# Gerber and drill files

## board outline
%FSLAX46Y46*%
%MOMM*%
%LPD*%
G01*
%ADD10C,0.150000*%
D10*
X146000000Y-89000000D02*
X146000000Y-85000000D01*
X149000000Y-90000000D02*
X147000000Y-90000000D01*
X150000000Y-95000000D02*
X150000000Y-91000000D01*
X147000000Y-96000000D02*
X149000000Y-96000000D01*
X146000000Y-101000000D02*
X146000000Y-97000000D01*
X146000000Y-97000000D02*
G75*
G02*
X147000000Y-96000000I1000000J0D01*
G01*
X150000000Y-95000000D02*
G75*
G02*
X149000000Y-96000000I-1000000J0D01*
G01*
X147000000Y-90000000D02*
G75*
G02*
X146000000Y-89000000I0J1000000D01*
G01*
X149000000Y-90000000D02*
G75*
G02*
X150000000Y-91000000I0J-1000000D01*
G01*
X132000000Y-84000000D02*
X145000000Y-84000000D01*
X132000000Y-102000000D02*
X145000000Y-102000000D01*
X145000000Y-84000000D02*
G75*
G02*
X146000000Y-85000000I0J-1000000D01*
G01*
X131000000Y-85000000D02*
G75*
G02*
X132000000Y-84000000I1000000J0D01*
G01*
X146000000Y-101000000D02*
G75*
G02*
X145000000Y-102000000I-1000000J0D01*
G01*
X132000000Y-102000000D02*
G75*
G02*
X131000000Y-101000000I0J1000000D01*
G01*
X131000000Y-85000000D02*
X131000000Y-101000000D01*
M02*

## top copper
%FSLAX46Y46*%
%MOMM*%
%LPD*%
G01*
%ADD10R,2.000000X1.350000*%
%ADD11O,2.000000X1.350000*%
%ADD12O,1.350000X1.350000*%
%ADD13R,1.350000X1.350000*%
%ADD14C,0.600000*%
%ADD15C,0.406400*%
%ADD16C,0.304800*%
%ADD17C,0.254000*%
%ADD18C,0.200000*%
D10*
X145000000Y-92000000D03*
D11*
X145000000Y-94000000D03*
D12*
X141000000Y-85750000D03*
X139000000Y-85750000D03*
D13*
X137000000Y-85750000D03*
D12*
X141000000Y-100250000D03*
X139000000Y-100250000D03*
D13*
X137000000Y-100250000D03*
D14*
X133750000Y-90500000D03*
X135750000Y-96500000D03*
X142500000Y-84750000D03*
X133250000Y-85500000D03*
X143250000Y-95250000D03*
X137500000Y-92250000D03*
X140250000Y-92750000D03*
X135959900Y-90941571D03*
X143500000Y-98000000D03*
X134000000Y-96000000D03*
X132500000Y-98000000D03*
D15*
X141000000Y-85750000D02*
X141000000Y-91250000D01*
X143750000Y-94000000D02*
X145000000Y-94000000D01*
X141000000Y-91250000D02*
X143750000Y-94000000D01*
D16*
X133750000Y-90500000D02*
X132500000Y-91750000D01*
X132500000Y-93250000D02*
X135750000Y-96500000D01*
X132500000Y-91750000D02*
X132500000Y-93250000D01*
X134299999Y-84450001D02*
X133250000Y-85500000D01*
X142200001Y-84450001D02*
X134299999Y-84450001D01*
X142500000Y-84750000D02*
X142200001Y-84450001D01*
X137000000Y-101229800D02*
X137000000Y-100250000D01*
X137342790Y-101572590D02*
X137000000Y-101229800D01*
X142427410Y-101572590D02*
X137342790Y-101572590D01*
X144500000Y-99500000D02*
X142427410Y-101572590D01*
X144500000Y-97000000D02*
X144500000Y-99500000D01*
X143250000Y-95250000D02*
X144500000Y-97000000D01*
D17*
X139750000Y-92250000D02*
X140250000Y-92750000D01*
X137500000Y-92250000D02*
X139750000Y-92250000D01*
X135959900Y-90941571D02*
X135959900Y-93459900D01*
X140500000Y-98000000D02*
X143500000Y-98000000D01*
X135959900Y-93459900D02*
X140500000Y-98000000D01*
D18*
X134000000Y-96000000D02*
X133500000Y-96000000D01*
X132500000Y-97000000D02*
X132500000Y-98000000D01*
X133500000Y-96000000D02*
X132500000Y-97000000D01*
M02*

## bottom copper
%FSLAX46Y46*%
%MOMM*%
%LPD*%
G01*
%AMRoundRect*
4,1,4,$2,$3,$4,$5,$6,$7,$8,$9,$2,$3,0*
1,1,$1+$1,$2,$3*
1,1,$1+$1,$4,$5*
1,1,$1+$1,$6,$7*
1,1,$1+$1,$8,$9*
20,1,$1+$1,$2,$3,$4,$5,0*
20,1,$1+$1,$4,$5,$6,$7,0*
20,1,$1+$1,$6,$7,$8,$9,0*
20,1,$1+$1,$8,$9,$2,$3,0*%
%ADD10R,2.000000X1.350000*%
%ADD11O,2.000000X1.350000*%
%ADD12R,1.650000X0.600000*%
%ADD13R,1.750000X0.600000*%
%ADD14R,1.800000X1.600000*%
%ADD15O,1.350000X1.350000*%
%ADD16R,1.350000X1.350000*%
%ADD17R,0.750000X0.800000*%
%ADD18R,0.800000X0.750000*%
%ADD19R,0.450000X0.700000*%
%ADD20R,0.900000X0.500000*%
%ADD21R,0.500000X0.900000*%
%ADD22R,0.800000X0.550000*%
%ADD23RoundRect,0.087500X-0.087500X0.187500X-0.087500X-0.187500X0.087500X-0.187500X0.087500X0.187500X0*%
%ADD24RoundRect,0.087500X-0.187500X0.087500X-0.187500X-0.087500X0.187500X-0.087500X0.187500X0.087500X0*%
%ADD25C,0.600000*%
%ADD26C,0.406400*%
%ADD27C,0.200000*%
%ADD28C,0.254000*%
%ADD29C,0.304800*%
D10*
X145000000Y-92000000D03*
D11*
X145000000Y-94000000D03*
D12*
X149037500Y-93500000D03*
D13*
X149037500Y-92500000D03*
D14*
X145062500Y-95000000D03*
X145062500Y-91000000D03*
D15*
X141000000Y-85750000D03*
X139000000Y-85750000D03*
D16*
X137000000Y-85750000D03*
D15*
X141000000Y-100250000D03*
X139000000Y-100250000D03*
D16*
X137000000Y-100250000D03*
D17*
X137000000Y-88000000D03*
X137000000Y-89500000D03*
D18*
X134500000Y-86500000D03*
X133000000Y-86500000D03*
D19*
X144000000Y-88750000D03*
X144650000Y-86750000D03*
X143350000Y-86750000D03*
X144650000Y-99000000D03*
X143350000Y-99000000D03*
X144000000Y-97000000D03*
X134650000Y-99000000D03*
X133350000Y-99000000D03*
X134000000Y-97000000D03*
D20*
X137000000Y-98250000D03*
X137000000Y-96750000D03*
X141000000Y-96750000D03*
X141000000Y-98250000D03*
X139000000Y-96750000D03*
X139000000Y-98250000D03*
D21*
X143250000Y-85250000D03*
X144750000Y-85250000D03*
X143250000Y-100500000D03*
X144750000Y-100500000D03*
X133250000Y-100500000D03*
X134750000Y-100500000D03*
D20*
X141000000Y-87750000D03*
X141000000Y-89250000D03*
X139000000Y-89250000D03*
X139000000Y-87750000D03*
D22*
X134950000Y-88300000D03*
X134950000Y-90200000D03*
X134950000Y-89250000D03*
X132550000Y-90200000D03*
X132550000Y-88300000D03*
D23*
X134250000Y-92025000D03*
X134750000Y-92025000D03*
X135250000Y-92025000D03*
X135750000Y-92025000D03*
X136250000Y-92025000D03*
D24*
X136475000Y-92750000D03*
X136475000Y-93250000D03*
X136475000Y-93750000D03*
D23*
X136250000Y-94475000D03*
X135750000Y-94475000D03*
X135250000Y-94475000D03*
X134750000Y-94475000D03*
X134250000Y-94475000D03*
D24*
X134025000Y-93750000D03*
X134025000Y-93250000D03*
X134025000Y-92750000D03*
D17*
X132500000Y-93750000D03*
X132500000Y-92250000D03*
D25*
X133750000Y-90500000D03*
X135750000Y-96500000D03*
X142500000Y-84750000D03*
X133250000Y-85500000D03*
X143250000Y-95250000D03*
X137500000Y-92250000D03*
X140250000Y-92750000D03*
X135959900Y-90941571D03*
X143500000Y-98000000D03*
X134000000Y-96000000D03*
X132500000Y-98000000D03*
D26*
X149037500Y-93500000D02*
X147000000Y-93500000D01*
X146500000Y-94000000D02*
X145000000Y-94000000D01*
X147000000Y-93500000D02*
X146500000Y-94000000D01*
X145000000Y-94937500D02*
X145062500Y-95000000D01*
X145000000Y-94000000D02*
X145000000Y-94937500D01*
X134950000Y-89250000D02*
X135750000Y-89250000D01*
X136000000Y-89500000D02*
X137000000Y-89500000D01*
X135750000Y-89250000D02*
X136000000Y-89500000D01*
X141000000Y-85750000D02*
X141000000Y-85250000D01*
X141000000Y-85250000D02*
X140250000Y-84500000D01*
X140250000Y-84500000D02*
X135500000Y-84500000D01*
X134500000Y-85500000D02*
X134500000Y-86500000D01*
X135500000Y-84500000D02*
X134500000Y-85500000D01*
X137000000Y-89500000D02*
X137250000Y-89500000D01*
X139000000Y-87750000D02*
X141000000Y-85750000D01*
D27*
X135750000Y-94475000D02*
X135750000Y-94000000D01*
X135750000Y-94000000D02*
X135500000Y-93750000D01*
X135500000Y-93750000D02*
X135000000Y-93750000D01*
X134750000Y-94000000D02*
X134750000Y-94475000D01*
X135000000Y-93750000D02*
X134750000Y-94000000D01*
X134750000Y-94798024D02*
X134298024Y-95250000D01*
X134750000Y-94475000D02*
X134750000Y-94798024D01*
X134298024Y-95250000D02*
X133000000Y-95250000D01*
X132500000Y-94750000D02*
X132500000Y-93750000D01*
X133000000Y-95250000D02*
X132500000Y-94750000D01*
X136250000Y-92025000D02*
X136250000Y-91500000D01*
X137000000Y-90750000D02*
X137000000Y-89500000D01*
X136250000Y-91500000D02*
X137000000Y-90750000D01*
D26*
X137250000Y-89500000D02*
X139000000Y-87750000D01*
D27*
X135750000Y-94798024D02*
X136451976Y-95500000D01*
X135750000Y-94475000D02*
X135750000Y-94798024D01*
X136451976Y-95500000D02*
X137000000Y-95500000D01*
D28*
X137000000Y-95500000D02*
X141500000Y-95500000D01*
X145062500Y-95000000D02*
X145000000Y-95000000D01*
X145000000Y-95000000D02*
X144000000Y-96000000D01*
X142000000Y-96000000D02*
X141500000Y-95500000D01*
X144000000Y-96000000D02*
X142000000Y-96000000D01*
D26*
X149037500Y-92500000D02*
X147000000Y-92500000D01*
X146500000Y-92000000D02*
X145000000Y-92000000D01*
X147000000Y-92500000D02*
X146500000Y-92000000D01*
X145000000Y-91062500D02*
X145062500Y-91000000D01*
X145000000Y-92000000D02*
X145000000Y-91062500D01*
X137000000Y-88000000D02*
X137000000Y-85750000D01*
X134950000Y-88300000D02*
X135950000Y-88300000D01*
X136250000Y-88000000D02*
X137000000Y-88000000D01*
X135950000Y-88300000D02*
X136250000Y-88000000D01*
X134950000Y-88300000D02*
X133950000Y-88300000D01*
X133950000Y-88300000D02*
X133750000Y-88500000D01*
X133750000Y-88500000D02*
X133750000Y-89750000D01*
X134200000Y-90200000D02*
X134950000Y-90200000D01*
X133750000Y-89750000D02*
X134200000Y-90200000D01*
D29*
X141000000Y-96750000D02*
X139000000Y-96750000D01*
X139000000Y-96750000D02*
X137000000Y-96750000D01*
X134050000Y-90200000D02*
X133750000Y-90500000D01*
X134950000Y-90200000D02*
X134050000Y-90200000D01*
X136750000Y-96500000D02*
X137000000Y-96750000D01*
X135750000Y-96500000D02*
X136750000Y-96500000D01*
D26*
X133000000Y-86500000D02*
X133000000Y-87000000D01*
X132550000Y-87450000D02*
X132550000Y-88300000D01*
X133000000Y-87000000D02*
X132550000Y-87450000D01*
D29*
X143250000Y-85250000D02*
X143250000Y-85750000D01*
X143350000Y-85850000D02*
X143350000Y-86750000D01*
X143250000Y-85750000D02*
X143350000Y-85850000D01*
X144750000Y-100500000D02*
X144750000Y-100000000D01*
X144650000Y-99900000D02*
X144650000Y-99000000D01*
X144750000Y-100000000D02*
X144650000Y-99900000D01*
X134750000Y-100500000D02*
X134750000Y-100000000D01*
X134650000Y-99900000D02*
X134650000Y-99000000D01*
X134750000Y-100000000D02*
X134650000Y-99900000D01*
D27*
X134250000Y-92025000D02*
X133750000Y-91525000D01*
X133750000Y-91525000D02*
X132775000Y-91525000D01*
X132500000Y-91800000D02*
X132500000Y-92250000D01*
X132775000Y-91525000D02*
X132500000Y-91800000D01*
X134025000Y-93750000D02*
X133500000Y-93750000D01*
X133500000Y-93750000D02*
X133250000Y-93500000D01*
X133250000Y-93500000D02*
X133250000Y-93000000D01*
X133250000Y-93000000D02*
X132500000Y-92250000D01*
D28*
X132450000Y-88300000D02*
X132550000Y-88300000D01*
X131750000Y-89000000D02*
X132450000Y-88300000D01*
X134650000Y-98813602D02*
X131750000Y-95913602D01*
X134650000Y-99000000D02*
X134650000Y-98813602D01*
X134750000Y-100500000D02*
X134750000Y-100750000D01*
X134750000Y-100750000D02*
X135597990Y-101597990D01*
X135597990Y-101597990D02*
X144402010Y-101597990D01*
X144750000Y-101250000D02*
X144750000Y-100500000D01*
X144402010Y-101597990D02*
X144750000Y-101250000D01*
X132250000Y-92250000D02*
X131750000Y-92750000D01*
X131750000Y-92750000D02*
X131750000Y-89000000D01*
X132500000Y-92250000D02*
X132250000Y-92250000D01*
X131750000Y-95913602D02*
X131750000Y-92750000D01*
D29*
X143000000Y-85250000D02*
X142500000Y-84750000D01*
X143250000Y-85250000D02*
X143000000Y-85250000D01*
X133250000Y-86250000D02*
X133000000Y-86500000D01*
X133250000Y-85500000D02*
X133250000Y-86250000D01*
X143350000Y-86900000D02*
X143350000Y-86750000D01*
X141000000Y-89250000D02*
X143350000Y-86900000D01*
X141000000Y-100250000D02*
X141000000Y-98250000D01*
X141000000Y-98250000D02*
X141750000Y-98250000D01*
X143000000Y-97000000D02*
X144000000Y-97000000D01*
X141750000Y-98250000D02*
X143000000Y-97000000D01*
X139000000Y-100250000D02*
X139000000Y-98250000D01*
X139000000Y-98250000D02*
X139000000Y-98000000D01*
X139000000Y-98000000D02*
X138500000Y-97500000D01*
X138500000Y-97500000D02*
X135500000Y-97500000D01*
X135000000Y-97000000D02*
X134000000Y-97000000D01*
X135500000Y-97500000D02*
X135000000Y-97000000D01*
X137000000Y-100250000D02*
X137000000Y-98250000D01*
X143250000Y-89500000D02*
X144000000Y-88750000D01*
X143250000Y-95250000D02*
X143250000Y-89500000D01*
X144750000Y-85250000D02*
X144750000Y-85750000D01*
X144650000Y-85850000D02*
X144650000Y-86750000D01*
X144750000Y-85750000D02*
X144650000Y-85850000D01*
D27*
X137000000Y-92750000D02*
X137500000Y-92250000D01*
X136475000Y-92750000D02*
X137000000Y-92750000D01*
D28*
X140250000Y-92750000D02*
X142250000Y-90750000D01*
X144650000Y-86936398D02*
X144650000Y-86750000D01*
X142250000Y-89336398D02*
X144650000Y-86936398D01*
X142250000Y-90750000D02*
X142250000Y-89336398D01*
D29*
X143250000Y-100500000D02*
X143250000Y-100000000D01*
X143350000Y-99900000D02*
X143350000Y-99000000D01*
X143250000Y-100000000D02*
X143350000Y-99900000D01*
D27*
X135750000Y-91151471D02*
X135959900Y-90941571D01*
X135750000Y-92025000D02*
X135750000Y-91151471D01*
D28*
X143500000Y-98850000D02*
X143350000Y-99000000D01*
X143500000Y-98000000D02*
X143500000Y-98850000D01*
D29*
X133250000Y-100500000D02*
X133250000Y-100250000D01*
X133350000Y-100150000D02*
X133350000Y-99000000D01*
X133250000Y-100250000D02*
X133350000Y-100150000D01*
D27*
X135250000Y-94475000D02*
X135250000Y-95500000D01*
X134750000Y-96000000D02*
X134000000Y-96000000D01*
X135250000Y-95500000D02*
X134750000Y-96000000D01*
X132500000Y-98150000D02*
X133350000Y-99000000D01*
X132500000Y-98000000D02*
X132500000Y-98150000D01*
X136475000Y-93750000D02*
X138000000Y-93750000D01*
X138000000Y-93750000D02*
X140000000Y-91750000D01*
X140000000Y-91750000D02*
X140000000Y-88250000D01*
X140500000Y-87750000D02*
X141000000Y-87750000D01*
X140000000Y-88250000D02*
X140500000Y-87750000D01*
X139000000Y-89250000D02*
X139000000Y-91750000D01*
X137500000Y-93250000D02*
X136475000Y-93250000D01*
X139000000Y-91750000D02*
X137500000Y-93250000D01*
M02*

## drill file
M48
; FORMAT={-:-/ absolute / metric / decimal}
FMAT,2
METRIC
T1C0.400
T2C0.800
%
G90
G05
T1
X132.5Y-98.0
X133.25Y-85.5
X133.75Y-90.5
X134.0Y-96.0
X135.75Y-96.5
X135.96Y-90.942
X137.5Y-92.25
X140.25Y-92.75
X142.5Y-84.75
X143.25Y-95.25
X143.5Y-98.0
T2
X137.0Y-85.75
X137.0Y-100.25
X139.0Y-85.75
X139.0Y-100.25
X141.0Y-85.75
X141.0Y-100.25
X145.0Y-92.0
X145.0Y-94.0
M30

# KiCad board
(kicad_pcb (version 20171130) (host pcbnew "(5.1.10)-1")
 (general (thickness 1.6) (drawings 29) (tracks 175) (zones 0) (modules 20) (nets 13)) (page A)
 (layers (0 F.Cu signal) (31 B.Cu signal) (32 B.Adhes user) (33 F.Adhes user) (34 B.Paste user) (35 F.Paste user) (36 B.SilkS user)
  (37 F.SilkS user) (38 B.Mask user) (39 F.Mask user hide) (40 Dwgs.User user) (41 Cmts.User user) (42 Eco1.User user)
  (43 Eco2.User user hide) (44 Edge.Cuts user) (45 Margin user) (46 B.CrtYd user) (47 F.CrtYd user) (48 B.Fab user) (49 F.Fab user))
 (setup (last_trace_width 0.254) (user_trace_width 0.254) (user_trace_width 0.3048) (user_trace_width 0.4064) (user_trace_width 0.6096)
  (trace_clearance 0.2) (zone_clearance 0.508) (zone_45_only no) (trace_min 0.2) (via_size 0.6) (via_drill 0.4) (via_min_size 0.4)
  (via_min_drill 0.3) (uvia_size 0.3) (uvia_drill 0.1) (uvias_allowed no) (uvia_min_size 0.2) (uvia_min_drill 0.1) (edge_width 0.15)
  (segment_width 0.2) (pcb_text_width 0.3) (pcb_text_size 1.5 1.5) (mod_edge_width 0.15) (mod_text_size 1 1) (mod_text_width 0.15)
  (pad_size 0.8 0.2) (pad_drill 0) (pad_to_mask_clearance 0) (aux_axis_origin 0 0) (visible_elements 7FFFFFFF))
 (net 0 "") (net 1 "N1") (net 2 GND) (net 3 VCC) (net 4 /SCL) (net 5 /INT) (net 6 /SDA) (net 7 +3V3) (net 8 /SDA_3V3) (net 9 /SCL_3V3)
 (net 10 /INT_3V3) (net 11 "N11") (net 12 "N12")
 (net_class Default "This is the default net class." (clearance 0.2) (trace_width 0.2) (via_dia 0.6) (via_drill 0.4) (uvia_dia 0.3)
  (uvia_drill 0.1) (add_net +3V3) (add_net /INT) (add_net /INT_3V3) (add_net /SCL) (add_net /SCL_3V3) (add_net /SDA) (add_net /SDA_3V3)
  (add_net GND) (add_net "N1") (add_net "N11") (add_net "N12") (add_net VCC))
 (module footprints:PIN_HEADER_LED (layer B.Cu) (at 145 92 180)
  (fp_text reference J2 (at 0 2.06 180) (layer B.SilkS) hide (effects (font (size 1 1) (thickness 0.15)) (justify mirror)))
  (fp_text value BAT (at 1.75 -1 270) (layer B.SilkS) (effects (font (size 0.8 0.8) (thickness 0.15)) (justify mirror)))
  (pad 1 thru_hole rect (at 0 0 180) (size 2 1.35) (drill 0.8) (layers *.Cu *.Mask) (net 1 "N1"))
  (pad 2 thru_hole oval (at 0 -2 180) (size 2 1.35) (drill 0.8) (layers *.Cu *.Mask) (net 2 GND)))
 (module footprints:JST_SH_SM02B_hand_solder (layer B.Cu) (at 147 93 90)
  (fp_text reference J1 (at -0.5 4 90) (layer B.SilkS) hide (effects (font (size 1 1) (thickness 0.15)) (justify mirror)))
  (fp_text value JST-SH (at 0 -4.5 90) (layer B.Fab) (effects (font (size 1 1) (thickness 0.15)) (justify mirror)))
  (pad 1 smd rect (at -0.5 2.0375 90) (size 0.6 1.65) (layers B.Cu B.Paste B.Mask) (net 2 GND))
  (pad 2 smd rect (at 0.5 2.0375 90) (size 0.6 1.75) (layers B.Cu B.Paste B.Mask) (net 1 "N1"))
  (pad 1 smd rect (at -2 -1.9375 90) (size 1.6 1.8) (layers B.Cu B.Paste B.Mask) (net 2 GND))
  (pad 2 smd rect (at 2 -1.9375 90) (size 1.6 1.8) (layers B.Cu B.Paste B.Mask) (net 1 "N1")))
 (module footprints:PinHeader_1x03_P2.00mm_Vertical (layer B.Cu) (at 137 85.75 270)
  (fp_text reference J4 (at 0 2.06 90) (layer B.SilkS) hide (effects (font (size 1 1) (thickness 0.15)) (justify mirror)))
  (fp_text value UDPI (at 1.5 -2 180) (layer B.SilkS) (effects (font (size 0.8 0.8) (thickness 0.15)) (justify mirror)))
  (pad 3 thru_hole oval (at 0 -4 270) (size 1.35 1.35) (drill 0.8) (layers *.Cu *.Mask) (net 2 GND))
  (pad 2 thru_hole oval (at 0 -2 270) (size 1.35 1.35) (drill 0.8) (layers *.Cu *.Mask))
  (pad 1 thru_hole rect (at 0 0 270) (size 1.35 1.35) (drill 0.8) (layers *.Cu *.Mask) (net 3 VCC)))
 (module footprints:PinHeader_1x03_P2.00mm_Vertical (layer B.Cu) (at 137 100.25 270)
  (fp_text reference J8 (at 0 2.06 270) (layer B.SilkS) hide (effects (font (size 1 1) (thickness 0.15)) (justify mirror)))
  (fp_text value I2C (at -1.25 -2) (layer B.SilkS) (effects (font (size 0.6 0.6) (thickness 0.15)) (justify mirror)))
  (pad 3 thru_hole oval (at 0 -4 270) (size 1.35 1.35) (drill 0.8) (layers *.Cu *.Mask) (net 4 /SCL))
  (pad 2 thru_hole oval (at 0 -2 270) (size 1.35 1.35) (drill 0.8) (layers *.Cu *.Mask) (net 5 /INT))
  (pad 1 thru_hole rect (at 0 0 270) (size 1.35 1.35) (drill 0.8) (layers *.Cu *.Mask) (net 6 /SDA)))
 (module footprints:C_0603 (layer B.Cu) (at 137 88.75 270)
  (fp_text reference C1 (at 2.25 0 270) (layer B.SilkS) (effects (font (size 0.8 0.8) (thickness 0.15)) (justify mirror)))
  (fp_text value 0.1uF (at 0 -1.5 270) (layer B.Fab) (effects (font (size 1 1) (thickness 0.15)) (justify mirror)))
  (pad 1 smd rect (at -0.75 0 270) (size 0.8 0.75) (layers B.Cu B.Paste B.Mask) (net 3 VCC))
  (pad 2 smd rect (at 0.75 0 270) (size 0.8 0.75) (layers B.Cu B.Paste B.Mask) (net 2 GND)))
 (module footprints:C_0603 (layer B.Cu) (at 133.75 86.5)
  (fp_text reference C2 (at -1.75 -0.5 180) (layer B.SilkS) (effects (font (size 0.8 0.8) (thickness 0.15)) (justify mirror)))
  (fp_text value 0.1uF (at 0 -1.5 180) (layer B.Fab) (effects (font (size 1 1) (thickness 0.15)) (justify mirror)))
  (pad 2 smd rect (at 0.75 0) (size 0.8 0.75) (layers B.Cu B.Paste B.Mask) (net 2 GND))
  (pad 1 smd rect (at -0.75 0) (size 0.8 0.75) (layers B.Cu B.Paste B.Mask) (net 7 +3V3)))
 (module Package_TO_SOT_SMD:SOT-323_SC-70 (layer B.Cu) (at 144 87.75 270)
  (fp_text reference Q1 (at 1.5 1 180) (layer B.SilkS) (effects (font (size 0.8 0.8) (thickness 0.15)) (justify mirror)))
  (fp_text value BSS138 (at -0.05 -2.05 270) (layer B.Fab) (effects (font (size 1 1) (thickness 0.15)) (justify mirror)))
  (pad 3 smd rect (at 1 0) (size 0.45 0.7) (layers B.Cu B.Paste B.Mask) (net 6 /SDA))
  (pad 2 smd rect (at -1 -0.65) (size 0.45 0.7) (layers B.Cu B.Paste B.Mask) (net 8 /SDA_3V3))
  (pad 1 smd rect (at -1 0.65) (size 0.45 0.7) (layers B.Cu B.Paste B.Mask) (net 7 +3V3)))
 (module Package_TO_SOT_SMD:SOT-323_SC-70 (layer B.Cu) (at 144 98 90)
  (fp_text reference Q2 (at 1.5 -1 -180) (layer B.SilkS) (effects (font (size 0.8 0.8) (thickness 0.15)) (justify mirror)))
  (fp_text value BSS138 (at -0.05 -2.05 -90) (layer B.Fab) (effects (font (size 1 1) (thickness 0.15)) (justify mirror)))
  (pad 1 smd rect (at -1 0.65 180) (size 0.45 0.7) (layers B.Cu B.Paste B.Mask) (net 7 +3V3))
  (pad 2 smd rect (at -1 -0.65 180) (size 0.45 0.7) (layers B.Cu B.Paste B.Mask) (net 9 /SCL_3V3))
  (pad 3 smd rect (at 1 0 180) (size 0.45 0.7) (layers B.Cu B.Paste B.Mask) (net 4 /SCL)))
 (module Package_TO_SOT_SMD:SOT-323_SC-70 (layer B.Cu) (at 134 98 90)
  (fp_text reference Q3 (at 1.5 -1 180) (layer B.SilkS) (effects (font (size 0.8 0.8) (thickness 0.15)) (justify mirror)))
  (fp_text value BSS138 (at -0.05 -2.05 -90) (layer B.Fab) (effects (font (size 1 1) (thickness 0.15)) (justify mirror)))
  (pad 1 smd rect (at -1 0.65 180) (size 0.45 0.7) (layers B.Cu B.Paste B.Mask) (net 7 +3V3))
  (pad 2 smd rect (at -1 -0.65 180) (size 0.45 0.7) (layers B.Cu B.Paste B.Mask) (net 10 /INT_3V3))
  (pad 3 smd rect (at 1 0 180) (size 0.45 0.7) (layers B.Cu B.Paste B.Mask) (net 5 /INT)))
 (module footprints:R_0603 (layer B.Cu) (at 137 97.5 270)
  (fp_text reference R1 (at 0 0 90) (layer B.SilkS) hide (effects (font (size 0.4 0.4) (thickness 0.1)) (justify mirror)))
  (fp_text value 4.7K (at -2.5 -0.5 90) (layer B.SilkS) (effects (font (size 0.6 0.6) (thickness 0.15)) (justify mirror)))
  (pad 2 smd rect (at 0.75 0 270) (size 0.5 0.9) (layers B.Cu B.Paste B.Mask) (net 6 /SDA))
  (pad 1 smd rect (at -0.75 0 270) (size 0.5 0.9) (layers B.Cu B.Paste B.Mask) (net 3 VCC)))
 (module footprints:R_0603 (layer B.Cu) (at 141 97.5 270)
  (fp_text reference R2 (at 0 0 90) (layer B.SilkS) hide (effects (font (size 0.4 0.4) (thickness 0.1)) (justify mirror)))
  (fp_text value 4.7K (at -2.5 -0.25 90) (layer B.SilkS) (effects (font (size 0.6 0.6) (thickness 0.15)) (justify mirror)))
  (pad 1 smd rect (at -0.75 0 270) (size 0.5 0.9) (layers B.Cu B.Paste B.Mask) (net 3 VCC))
  (pad 2 smd rect (at 0.75 0 270) (size 0.5 0.9) (layers B.Cu B.Paste B.Mask) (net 4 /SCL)))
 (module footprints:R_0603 (layer B.Cu) (at 139 97.5 270)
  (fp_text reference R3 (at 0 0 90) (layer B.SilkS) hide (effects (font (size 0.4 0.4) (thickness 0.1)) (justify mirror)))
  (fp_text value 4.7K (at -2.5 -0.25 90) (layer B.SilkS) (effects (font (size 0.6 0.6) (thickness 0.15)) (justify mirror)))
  (pad 1 smd rect (at -0.75 0 270) (size 0.5 0.9) (layers B.Cu B.Paste B.Mask) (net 3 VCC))
  (pad 2 smd rect (at 0.75 0 270) (size 0.5 0.9) (layers B.Cu B.Paste B.Mask) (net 5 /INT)))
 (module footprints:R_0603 (layer B.Cu) (at 144 85.25)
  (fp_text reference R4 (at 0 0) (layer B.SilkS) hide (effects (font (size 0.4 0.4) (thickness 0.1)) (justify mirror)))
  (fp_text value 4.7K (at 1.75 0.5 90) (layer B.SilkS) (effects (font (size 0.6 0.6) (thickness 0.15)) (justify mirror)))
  (pad 1 smd rect (at -0.75 0) (size 0.5 0.9) (layers B.Cu B.Paste B.Mask) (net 7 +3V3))
  (pad 2 smd rect (at 0.75 0) (size 0.5 0.9) (layers B.Cu B.Paste B.Mask) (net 8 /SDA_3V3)))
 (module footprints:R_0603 (layer B.Cu) (at 144 100.5 180)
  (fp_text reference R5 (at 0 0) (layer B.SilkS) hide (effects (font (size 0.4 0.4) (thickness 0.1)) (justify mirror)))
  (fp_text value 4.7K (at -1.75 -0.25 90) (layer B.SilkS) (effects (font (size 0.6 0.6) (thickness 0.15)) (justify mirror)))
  (pad 2 smd rect (at 0.75 0 180) (size 0.5 0.9) (layers B.Cu B.Paste B.Mask) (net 9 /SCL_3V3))
  (pad 1 smd rect (at -0.75 0 180) (size 0.5 0.9) (layers B.Cu B.Paste B.Mask) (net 7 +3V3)))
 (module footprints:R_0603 (layer B.Cu) (at 134 100.5 180)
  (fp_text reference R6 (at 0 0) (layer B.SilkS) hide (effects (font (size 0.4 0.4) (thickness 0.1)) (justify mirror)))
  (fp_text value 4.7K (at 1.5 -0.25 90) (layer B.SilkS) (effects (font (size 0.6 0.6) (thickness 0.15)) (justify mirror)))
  (pad 2 smd rect (at 0.75 0 180) (size 0.5 0.9) (layers B.Cu B.Paste B.Mask) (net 10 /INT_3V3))
  (pad 1 smd rect (at -0.75 0 180) (size 0.5 0.9) (layers B.Cu B.Paste B.Mask) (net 7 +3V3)))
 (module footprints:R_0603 (layer B.Cu) (at 141 88.5 90)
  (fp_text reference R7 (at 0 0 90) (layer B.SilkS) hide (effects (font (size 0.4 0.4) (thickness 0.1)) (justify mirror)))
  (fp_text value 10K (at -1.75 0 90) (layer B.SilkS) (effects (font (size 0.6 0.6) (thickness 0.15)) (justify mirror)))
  (pad 2 smd rect (at 0.75 0 90) (size 0.5 0.9) (layers B.Cu B.Paste B.Mask) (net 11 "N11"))
  (pad 1 smd rect (at -0.75 0 90) (size 0.5 0.9) (layers B.Cu B.Paste B.Mask) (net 7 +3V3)))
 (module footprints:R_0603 (layer B.Cu) (at 139 88.5 90)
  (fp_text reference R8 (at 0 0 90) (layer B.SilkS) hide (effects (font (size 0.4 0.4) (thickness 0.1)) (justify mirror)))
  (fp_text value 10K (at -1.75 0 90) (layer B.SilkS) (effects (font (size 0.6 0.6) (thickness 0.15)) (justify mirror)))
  (pad 1 smd rect (at -0.75 0 90) (size 0.5 0.9) (layers B.Cu B.Paste B.Mask) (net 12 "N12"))
  (pad 2 smd rect (at 0.75 0 90) (size 0.5 0.9) (layers B.Cu B.Paste B.Mask) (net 2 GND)))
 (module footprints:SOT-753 (layer B.Cu) (at 133.75 89.25 270) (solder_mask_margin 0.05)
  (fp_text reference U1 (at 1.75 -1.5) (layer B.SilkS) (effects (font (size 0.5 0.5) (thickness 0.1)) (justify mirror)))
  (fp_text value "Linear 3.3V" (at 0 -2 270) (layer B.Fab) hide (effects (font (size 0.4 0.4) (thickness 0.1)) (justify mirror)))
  (pad 1 smd rect (at -0.95 -1.2 270) (size 0.55 0.8) (layers B.Cu B.Paste B.Mask) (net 3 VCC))
  (pad 3 smd rect (at 0.95 -1.2 270) (size 0.55 0.8) (layers B.Cu B.Paste B.Mask) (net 3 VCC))
  (pad 2 smd rect (at 0 -1.2 270) (size 0.55 0.8) (layers B.Cu B.Paste B.Mask) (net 2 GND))
  (pad 4 smd rect (at 0.95 1.2 270) (size 0.55 0.8) (layers B.Cu B.Paste B.Mask))
  (pad 5 smd rect (at -0.95 1.2 270) (size 0.55 0.8) (layers B.Cu B.Paste B.Mask) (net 7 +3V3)))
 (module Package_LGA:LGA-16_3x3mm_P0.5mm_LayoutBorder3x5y (layer B.Cu) (at 135.25 93.25 270)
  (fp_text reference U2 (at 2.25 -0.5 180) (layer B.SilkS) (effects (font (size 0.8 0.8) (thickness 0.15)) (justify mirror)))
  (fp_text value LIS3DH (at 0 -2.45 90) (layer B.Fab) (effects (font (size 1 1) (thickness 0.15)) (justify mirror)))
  (pad 1 smd roundrect (at -1.225 1 270) (size 0.55 0.35) (layers B.Cu B.Paste B.Mask) (roundrect_rratio 0.25) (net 7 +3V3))
  (pad 2 smd roundrect (at -1.225 0.5 270) (size 0.55 0.35) (layers B.Cu B.Paste B.Mask) (roundrect_rratio 0.25))
  (pad 3 smd roundrect (at -1.225 0 270) (size 0.55 0.35) (layers B.Cu B.Paste B.Mask) (roundrect_rratio 0.25))
  (pad 4 smd roundrect (at -1.225 -0.5 270) (size 0.55 0.35) (layers B.Cu B.Paste B.Mask) (roundrect_rratio 0.25) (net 9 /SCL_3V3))
  (pad 5 smd roundrect (at -1.225 -1 270) (size 0.55 0.35) (layers B.Cu B.Paste B.Mask) (roundrect_rratio 0.25) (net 2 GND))
  (pad 6 smd roundrect (at -0.5 -1.225 270) (size 0.35 0.55) (layers B.Cu B.Paste B.Mask) (roundrect_rratio 0.25) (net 8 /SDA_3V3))
  (pad 7 smd roundrect (at 0 -1.225 270) (size 0.35 0.55) (layers B.Cu B.Paste B.Mask) (roundrect_rratio 0.25) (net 12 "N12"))
  (pad 8 smd roundrect (at 0.5 -1.225 270) (size 0.35 0.55) (layers B.Cu B.Paste B.Mask) (roundrect_rratio 0.25) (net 11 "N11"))
  (pad 9 smd roundrect (at 1.225 -1 270) (size 0.55 0.35) (layers B.Cu B.Paste B.Mask) (roundrect_rratio 0.25))
  (pad 10 smd roundrect (at 1.225 -0.5 270) (size 0.55 0.35) (layers B.Cu B.Paste B.Mask) (roundrect_rratio 0.25) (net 2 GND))
  (pad 11 smd roundrect (at 1.225 0 270) (size 0.55 0.35) (layers B.Cu B.Paste B.Mask) (roundrect_rratio 0.25) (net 10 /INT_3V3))
  (pad 12 smd roundrect (at 1.225 0.5 270) (size 0.55 0.35) (layers B.Cu B.Paste B.Mask) (roundrect_rratio 0.25) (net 2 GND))
  (pad 13 smd roundrect (at 1.225 1 270) (size 0.55 0.35) (layers B.Cu B.Paste B.Mask) (roundrect_rratio 0.25))
  (pad 14 smd roundrect (at 0.5 1.225 270) (size 0.35 0.55) (layers B.Cu B.Paste B.Mask) (roundrect_rratio 0.25) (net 7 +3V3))
  (pad 15 smd roundrect (at 0 1.225 270) (size 0.35 0.55) (layers B.Cu B.Paste B.Mask) (roundrect_rratio 0.25))
  (pad 16 smd roundrect (at -0.5 1.225 270) (size 0.35 0.55) (layers B.Cu B.Paste B.Mask) (roundrect_rratio 0.25)))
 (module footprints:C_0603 (layer B.Cu) (at 132.5 93 270)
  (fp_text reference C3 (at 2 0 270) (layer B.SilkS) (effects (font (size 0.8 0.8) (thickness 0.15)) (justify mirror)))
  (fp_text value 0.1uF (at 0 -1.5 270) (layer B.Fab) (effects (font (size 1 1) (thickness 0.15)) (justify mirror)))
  (pad 2 smd rect (at 0.75 0 270) (size 0.8 0.75) (layers B.Cu B.Paste B.Mask) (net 2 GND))
  (pad 1 smd rect (at -0.75 0 270) (size 0.8 0.75) (layers B.Cu B.Paste B.Mask) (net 7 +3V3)))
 (gr_line (start 146 89) (end 146 85) (layer Edge.Cuts) (width 0.15))
 (gr_line (start 149 90) (end 147 90) (layer Edge.Cuts) (width 0.15))
 (gr_line (start 150 95) (end 150 91) (layer Edge.Cuts) (width 0.15))
 (gr_line (start 147 96) (end 149 96) (layer Edge.Cuts) (width 0.15))
 (gr_line (start 146 101) (end 146 97) (layer Edge.Cuts) (width 0.15))
 (gr_arc (start 147 97) (end 147 96) (angle -90) (layer Edge.Cuts) (width 0.15))
 (gr_arc (start 149 95) (end 149 96) (angle -90) (layer Edge.Cuts) (width 0.15))
 (gr_arc (start 147 89) (end 146 89) (angle -90) (layer Edge.Cuts) (width 0.15))
 (gr_arc (start 149 91) (end 150 91) (angle -90) (layer Edge.Cuts) (width 0.15))
 (gr_line (start 132 84) (end 145 84) (layer Edge.Cuts) (width 0.15))
 (gr_line (start 132 102) (end 145 102) (layer Edge.Cuts) (width 0.15))
 (gr_arc (start 145 85) (end 145 84) (angle 90) (layer Edge.Cuts) (width 0.15))
 (gr_arc (start 132 85) (end 131 85) (angle 90) (layer Edge.Cuts) (width 0.15))
 (gr_arc (start 145 101) (end 146 101) (angle 90) (layer Edge.Cuts) (width 0.15))
 (gr_arc (start 132 101) (end 132 102) (angle 90) (layer Edge.Cuts) (width 0.15))
 (gr_line (start 131 85) (end 131 101) (angle 90) (layer Edge.Cuts) (width 0.15))
 (segment (start 149.0375 93.5) (end 147 93.5) (width 0.4064) (layer B.Cu) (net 2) (status 10))
 (segment (start 146.5 94) (end 145 94) (width 0.4064) (layer B.Cu) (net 2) (status 20))
 (segment (start 147 93.5) (end 146.5 94) (width 0.4064) (layer B.Cu) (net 2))
 (segment (start 145 94.9375) (end 145.0625 95) (width 0.4064) (layer B.Cu) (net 2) (status 30))
 (segment (start 145 94) (end 145 94.9375) (width 0.4064) (layer B.Cu) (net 2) (status 30))
 (segment (start 134.95 89.25) (end 135.75 89.25) (width 0.4064) (layer B.Cu) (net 2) (status 10))
 (segment (start 136 89.5) (end 137 89.5) (width 0.4064) (layer B.Cu) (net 2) (status 20))
 (segment (start 135.75 89.25) (end 136 89.5) (width 0.4064) (layer B.Cu) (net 2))
 (segment (start 141 85.75) (end 141 85.25) (width 0.4064) (layer B.Cu) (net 2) (status 30))
 (segment (start 141 85.25) (end 140.25 84.5) (width 0.4064) (layer B.Cu) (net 2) (status 10))
 (segment (start 140.25 84.5) (end 135.5 84.5) (width 0.4064) (layer B.Cu) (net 2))
 (segment (start 134.5 85.5) (end 134.5 86.5) (width 0.4064) (layer B.Cu) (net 2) (status 20))
 (segment (start 135.5 84.5) (end 134.5 85.5) (width 0.4064) (layer B.Cu) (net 2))
 (segment (start 137 89.5) (end 137.25 89.5) (width 0.4064) (layer B.Cu) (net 2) (status 30))
 (segment (start 139 87.75) (end 141 85.75) (width 0.4064) (layer B.Cu) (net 2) (status 30))
 (segment (start 135.75 94.475) (end 135.75 94) (width 0.2) (layer B.Cu) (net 2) (status 10))
 (segment (start 135.75 94) (end 135.5 93.75) (width 0.2) (layer B.Cu) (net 2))
 (segment (start 135.5 93.75) (end 135 93.75) (width 0.2) (layer B.Cu) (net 2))
 (segment (start 134.75 94) (end 134.75 94.475) (width 0.2) (layer B.Cu) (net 2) (status 20))
 (segment (start 135 93.75) (end 134.75 94) (width 0.2) (layer B.Cu) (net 2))
 (segment (start 134.75 94.798024) (end 134.298024 95.25) (width 0.2) (layer B.Cu) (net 2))
 (segment (start 134.75 94.475) (end 134.75 94.798024) (width 0.2) (layer B.Cu) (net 2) (status 10))
 (segment (start 134.298024 95.25) (end 133 95.25) (width 0.2) (layer B.Cu) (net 2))
 (segment (start 132.5 94.75) (end 132.5 93.75) (width 0.2) (layer B.Cu) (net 2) (status 20))
 (segment (start 133 95.25) (end 132.5 94.75) (width 0.2) (layer B.Cu) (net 2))
 (segment (start 141 85.75) (end 141 91.25) (width 0.4064) (layer F.Cu) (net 2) (status 10))
 (segment (start 143.75 94) (end 145 94) (width 0.4064) (layer F.Cu) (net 2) (status 20))
 (segment (start 141 91.25) (end 143.75 94) (width 0.4064) (layer F.Cu) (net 2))
 (segment (start 136.25 92.025) (end 136.25 91.5) (width 0.2) (layer B.Cu) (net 2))
 (segment (start 137 90.75) (end 137 89.5) (width 0.2) (layer B.Cu) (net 2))
 (segment (start 136.25 91.5) (end 137 90.75) (width 0.2) (layer B.Cu) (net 2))
 (segment (start 137.25 89.5) (end 139 87.75) (width 0.4064) (layer B.Cu) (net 2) (status 30))
 (segment (start 135.75 94.798024) (end 136.451976 95.5) (width 0.2) (layer B.Cu) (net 2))
 (segment (start 135.75 94.475) (end 135.75 94.798024) (width 0.2) (layer B.Cu) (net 2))
 (segment (start 136.451976 95.5) (end 137 95.5) (width 0.2) (layer B.Cu) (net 2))
 (segment (start 137 95.5) (end 141.5 95.5) (width 0.254) (layer B.Cu) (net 2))
 (segment (start 145.0625 95) (end 145 95) (width 0.254) (layer B.Cu) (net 2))
 (segment (start 145 95) (end 144 96) (width 0.254) (layer B.Cu) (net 2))
 (segment (start 142 96) (end 141.5 95.5) (width 0.254) (layer B.Cu) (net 2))
 (segment (start 144 96) (end 142 96) (width 0.254) (layer B.Cu) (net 2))
 (segment (start 149.0375 92.5) (end 147 92.5) (width 0.4064) (layer B.Cu) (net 1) (status 10))
 (segment (start 146.5 92) (end 145 92) (width 0.4064) (layer B.Cu) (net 1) (status 20))
 (segment (start 147 92.5) (end 146.5 92) (width 0.4064) (layer B.Cu) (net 1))
 (segment (start 145 91.0625) (end 145.0625 91) (width 0.4064) (layer B.Cu) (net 1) (status 30))
 (segment (start 145 92) (end 145 91.0625) (width 0.4064) (layer B.Cu) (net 1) (status 30))
 (segment (start 137 88) (end 137 85.75) (width 0.4064) (layer B.Cu) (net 3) (status 30))
 (segment (start 134.95 88.3) (end 135.95 88.3) (width 0.4064) (layer B.Cu) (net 3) (status 10))
 (segment (start 136.25 88) (end 137 88) (width 0.4064) (layer B.Cu) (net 3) (status 20))
 (segment (start 135.95 88.3) (end 136.25 88) (width 0.4064) (layer B.Cu) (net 3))
 (segment (start 134.95 88.3) (end 133.95 88.3) (width 0.4064) (layer B.Cu) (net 3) (status 10))
 (segment (start 133.95 88.3) (end 133.75 88.5) (width 0.4064) (layer B.Cu) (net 3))
 (segment (start 133.75 88.5) (end 133.75 89.75) (width 0.4064) (layer B.Cu) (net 3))
 (segment (start 134.2 90.2) (end 134.95 90.2) (width 0.4064) (layer B.Cu) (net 3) (status 20))
 (segment (start 133.75 89.75) (end 134.2 90.2) (width 0.4064) (layer B.Cu) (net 3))
 (segment (start 141 96.75) (end 139 96.75) (width 0.3048) (layer B.Cu) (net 3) (status 30))
 (segment (start 139 96.75) (end 137 96.75) (width 0.3048) (layer B.Cu) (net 3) (status 30))
 (via (at 133.75 90.5) (size 0.6) (drill 0.4) (layers F.Cu B.Cu) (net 3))
 (segment (start 134.05 90.2) (end 133.75 90.5) (width 0.3048) (layer B.Cu) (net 3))
 (segment (start 134.95 90.2) (end 134.05 90.2) (width 0.3048) (layer B.Cu) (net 3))
 (segment (start 133.75 90.5) (end 132.5 91.75) (width 0.3048) (layer F.Cu) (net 3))
 (via (at 135.75 96.5) (size 0.6) (drill 0.4) (layers F.Cu B.Cu) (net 3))
 (segment (start 132.5 93.25) (end 135.75 96.5) (width 0.3048) (layer F.Cu) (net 3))
 (segment (start 132.5 91.75) (end 132.5 93.25) (width 0.3048) (layer F.Cu) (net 3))
 (segment (start 136.75 96.5) (end 137 96.75) (width 0.3048) (layer B.Cu) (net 3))
 (segment (start 135.75 96.5) (end 136.75 96.5) (width 0.3048) (layer B.Cu) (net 3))
 (segment (start 133 86.5) (end 133 87) (width 0.4064) (layer B.Cu) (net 7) (status 10))
 (segment (start 132.55 87.45) (end 132.55 88.3) (width 0.4064) (layer B.Cu) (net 7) (status 20))
 (segment (start 133 87) (end 132.55 87.45) (width 0.4064) (layer B.Cu) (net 7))
 (segment (start 143.25 85.25) (end 143.25 85.75) (width 0.3048) (layer B.Cu) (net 7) (status 10))
 (segment (start 143.35 85.85) (end 143.35 86.75) (width 0.3048) (layer B.Cu) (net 7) (status 20))
 (segment (start 143.25 85.75) (end 143.35 85.85) (width 0.3048) (layer B.Cu) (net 7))
 (segment (start 144.75 100.5) (end 144.75 100) (width 0.3048) (layer B.Cu) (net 7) (status 10))
 (segment (start 144.65 99.9) (end 144.65 99) (width 0.3048) (layer B.Cu) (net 7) (status 20))
 (segment (start 144.75 100) (end 144.65 99.9) (width 0.3048) (layer B.Cu) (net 7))
 (segment (start 134.75 100.5) (end 134.75 100) (width 0.3048) (layer B.Cu) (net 7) (status 10))
 (segment (start 134.65 99.9) (end 134.65 99) (width 0.3048) (layer B.Cu) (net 7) (status 20))
 (segment (start 134.75 100) (end 134.65 99.9) (width 0.3048) (layer B.Cu) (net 7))
 (segment (start 134.25 92.025) (end 133.75 91.525) (width 0.2) (layer B.Cu) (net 7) (status 10))
 (segment (start 133.75 91.525) (end 132.775 91.525) (width 0.2) (layer B.Cu) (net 7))
 (segment (start 132.5 91.8) (end 132.5 92.25) (width 0.2) (layer B.Cu) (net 7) (status 20))
 (segment (start 132.775 91.525) (end 132.5 91.8) (width 0.2) (layer B.Cu) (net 7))
 (segment (start 134.025 93.75) (end 133.5 93.75) (width 0.2) (layer B.Cu) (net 7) (status 10))
 (segment (start 133.5 93.75) (end 133.25 93.5) (width 0.2) (layer B.Cu) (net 7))
 (segment (start 133.25 93.5) (end 133.25 93) (width 0.2) (layer B.Cu) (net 7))
 (segment (start 133.25 93) (end 132.5 92.25) (width 0.2) (layer B.Cu) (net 7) (status 20))
 (segment (start 132.45 88.3) (end 132.55 88.3) (width 0.254) (layer B.Cu) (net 7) (status 30))
 (segment (start 131.75 89) (end 132.45 88.3) (width 0.254) (layer B.Cu) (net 7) (status 20))
 (segment (start 134.65 98.813602) (end 131.75 95.913602) (width 0.254) (layer B.Cu) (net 7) (status 10))
 (segment (start 134.65 99) (end 134.65 98.813602) (width 0.254) (layer B.Cu) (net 7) (status 30))
 (segment (start 134.75 100.5) (end 134.75 100.75) (width 0.254) (layer B.Cu) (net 7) (status 30))
 (segment (start 134.75 100.75) (end 135.59799 101.59799) (width 0.254) (layer B.Cu) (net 7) (status 10))
 (segment (start 135.59799 101.59799) (end 144.40201 101.59799) (width 0.254) (layer B.Cu) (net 7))
 (segment (start 144.75 101.25) (end 144.75 100.5) (width 0.254) (layer B.Cu) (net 7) (status 20))
 (segment (start 144.40201 101.59799) (end 144.75 101.25) (width 0.254) (layer B.Cu) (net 7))
 (segment (start 132.25 92.25) (end 131.75 92.75) (width 0.254) (layer B.Cu) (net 7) (status 10))
 (segment (start 131.75 92.75) (end 131.75 89) (width 0.254) (layer B.Cu) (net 7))
 (segment (start 132.5 92.25) (end 132.25 92.25) (width 0.254) (layer B.Cu) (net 7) (status 30))
 (segment (start 131.75 95.913602) (end 131.75 92.75) (width 0.254) (layer B.Cu) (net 7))
 (via (at 142.5 84.75) (size 0.6) (drill 0.4) (layers F.Cu B.Cu) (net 7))
 (segment (start 143 85.25) (end 142.5 84.75) (width 0.3048) (layer B.Cu) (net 7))
 (segment (start 143.25 85.25) (end 143 85.25) (width 0.3048) (layer B.Cu) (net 7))
 (via (at 133.25 85.5) (size 0.6) (drill 0.4) (layers F.Cu B.Cu) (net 7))
 (segment (start 134.299999 84.450001) (end 133.25 85.5) (width 0.3048) (layer F.Cu) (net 7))
 (segment (start 142.200001 84.450001) (end 134.299999 84.450001) (width 0.3048) (layer F.Cu) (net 7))
 (segment (start 142.5 84.75) (end 142.200001 84.450001) (width 0.3048) (layer F.Cu) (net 7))
 (segment (start 133.25 86.25) (end 133 86.5) (width 0.3048) (layer B.Cu) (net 7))
 (segment (start 133.25 85.5) (end 133.25 86.25) (width 0.3048) (layer B.Cu) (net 7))
 (segment (start 143.35 86.9) (end 143.35 86.75) (width 0.3048) (layer B.Cu) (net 7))
 (segment (start 141 89.25) (end 143.35 86.9) (width 0.3048) (layer B.Cu) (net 7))
 (segment (start 141 100.25) (end 141 98.25) (width 0.3048) (layer B.Cu) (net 4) (status 30))
 (segment (start 141 98.25) (end 141.75 98.25) (width 0.3048) (layer B.Cu) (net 4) (status 10))
 (segment (start 143 97) (end 144 97) (width 0.3048) (layer B.Cu) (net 4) (status 20))
 (segment (start 141.75 98.25) (end 143 97) (width 0.3048) (layer B.Cu) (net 4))
 (segment (start 139 100.25) (end 139 98.25) (width 0.3048) (layer B.Cu) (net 5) (status 30))
 (segment (start 139 98.25) (end 139 98) (width 0.3048) (layer B.Cu) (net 5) (status 30))
 (segment (start 139 98) (end 138.5 97.5) (width 0.3048) (layer B.Cu) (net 5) (status 10))
 (segment (start 138.5 97.5) (end 135.5 97.5) (width 0.3048) (layer B.Cu) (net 5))
 (segment (start 135 97) (end 134 97) (width 0.3048) (layer B.Cu) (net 5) (status 20))
 (segment (start 135.5 97.5) (end 135 97) (width 0.3048) (layer B.Cu) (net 5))
 (segment (start 137 100.25) (end 137 98.25) (width 0.3048) (layer B.Cu) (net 6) (status 30))
 (segment (start 143.25 89.5) (end 144 88.75) (width 0.3048) (layer B.Cu) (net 6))
 (segment (start 143.25 95.25) (end 143.25 89.5) (width 0.3048) (layer B.Cu) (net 6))
 (segment (start 137 101.2298) (end 137 100.25) (width 0.3048) (layer F.Cu) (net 6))
 (segment (start 137.34279 101.57259) (end 137 101.2298) (width 0.3048) (layer F.Cu) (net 6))
 (segment (start 142.42741 101.57259) (end 137.34279 101.57259) (width 0.3048) (layer F.Cu) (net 6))
 (segment (start 144.5 99.5) (end 142.42741 101.57259) (width 0.3048) (layer F.Cu) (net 6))
 (segment (start 144.5 97) (end 144.5 99.5) (width 0.3048) (layer F.Cu) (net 6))
 (segment (start 143.25 95.25) (end 144.5 97) (width 0.3048) (layer F.Cu) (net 6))
 (via (at 143.25 95.25) (size 0.6) (drill 0.4) (layers F.Cu B.Cu) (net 6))
 (segment (start 144.75 85.25) (end 144.75 85.75) (width 0.3048) (layer B.Cu) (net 8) (status 10))
 (segment (start 144.65 85.85) (end 144.65 86.75) (width 0.3048) (layer B.Cu) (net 8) (status 20))
 (segment (start 144.75 85.75) (end 144.65 85.85) (width 0.3048) (layer B.Cu) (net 8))
 (via (at 137.5 92.25) (size 0.6) (drill 0.4) (layers F.Cu B.Cu) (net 8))
 (segment (start 137 92.75) (end 137.5 92.25) (width 0.2) (layer B.Cu) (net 8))
 (segment (start 136.475 92.75) (end 137 92.75) (width 0.2) (layer B.Cu) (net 8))
 (via (at 140.25 92.75) (size 0.6) (drill 0.4) (layers F.Cu B.Cu) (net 8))
 (segment (start 139.75 92.25) (end 140.25 92.75) (width 0.254) (layer F.Cu) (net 8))
 (segment (start 137.5 92.25) (end 139.75 92.25) (width 0.254) (layer F.Cu) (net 8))
 (segment (start 140.25 92.75) (end 142.25 90.75) (width 0.254) (layer B.Cu) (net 8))
 (segment (start 144.65 86.936398) (end 144.65 86.75) (width 0.254) (layer B.Cu) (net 8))
 (segment (start 142.25 89.336398) (end 144.65 86.936398) (width 0.254) (layer B.Cu) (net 8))
 (segment (start 142.25 90.75) (end 142.25 89.336398) (width 0.254) (layer B.Cu) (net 8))
 (segment (start 143.25 100.5) (end 143.25 100) (width 0.3048) (layer B.Cu) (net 9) (status 10))
 (segment (start 143.35 99.9) (end 143.35 99) (width 0.3048) (layer B.Cu) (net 9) (status 20))
 (segment (start 143.25 100) (end 143.35 99.9) (width 0.3048) (layer B.Cu) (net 9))
 (via (at 135.9599 90.941571) (size 0.6) (drill 0.4) (layers F.Cu B.Cu) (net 9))
 (segment (start 135.75 91.151471) (end 135.9599 90.941571) (width 0.2) (layer B.Cu) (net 9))
 (segment (start 135.75 92.025) (end 135.75 91.151471) (width 0.2) (layer B.Cu) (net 9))
 (segment (start 135.9599 90.941571) (end 135.9599 93.4599) (width 0.254) (layer F.Cu) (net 9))
 (via (at 143.5 98) (size 0.6) (drill 0.4) (layers F.Cu B.Cu) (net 9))
 (segment (start 140.5 98) (end 143.5 98) (width 0.254) (layer F.Cu) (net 9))
 (segment (start 135.9599 93.4599) (end 140.5 98) (width 0.254) (layer F.Cu) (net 9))
 (segment (start 143.5 98.85) (end 143.35 99) (width 0.254) (layer B.Cu) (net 9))
 (segment (start 143.5 98) (end 143.5 98.85) (width 0.254) (layer B.Cu) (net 9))
 (segment (start 133.25 100.5) (end 133.25 100.25) (width 0.3048) (layer B.Cu) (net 10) (status 30))
 (segment (start 133.35 100.15) (end 133.35 99) (width 0.3048) (layer B.Cu) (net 10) (status 30))
 (segment (start 133.25 100.25) (end 133.35 100.15) (width 0.3048) (layer B.Cu) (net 10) (status 30))
 (segment (start 135.25 94.475) (end 135.25 95.5) (width 0.2) (layer B.Cu) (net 10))
 (via (at 134 96) (size 0.6) (drill 0.4) (layers F.Cu B.Cu) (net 10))
 (segment (start 134.75 96) (end 134 96) (width 0.2) (layer B.Cu) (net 10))
 (segment (start 135.25 95.5) (end 134.75 96) (width 0.2) (layer B.Cu) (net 10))
 (segment (start 134 96) (end 133.5 96) (width 0.2) (layer F.Cu) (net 10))
 (via (at 132.5 98) (size 0.6) (drill 0.4) (layers F.Cu B.Cu) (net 10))
 (segment (start 132.5 97) (end 132.5 98) (width 0.2) (layer F.Cu) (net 10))
 (segment (start 133.5 96) (end 132.5 97) (width 0.2) (layer F.Cu) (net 10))
 (segment (start 132.5 98.15) (end 133.35 99) (width 0.2) (layer B.Cu) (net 10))
 (segment (start 132.5 98) (end 132.5 98.15) (width 0.2) (layer B.Cu) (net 10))
 (segment (start 136.475 93.75) (end 138 93.75) (width 0.2) (layer B.Cu) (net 11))
 (segment (start 138 93.75) (end 140 91.75) (width 0.2) (layer B.Cu) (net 11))
 (segment (start 140 91.75) (end 140 88.25) (width 0.2) (layer B.Cu) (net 11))
 (segment (start 140.5 87.75) (end 141 87.75) (width 0.2) (layer B.Cu) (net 11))
 (segment (start 140 88.25) (end 140.5 87.75) (width 0.2) (layer B.Cu) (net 11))
 (segment (start 139 89.25) (end 139 91.75) (width 0.2) (layer B.Cu) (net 12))
 (segment (start 137.5 93.25) (end 136.475 93.25) (width 0.2) (layer B.Cu) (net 12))
 (segment (start 139 91.75) (end 137.5 93.25) (width 0.2) (layer B.Cu) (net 12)))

